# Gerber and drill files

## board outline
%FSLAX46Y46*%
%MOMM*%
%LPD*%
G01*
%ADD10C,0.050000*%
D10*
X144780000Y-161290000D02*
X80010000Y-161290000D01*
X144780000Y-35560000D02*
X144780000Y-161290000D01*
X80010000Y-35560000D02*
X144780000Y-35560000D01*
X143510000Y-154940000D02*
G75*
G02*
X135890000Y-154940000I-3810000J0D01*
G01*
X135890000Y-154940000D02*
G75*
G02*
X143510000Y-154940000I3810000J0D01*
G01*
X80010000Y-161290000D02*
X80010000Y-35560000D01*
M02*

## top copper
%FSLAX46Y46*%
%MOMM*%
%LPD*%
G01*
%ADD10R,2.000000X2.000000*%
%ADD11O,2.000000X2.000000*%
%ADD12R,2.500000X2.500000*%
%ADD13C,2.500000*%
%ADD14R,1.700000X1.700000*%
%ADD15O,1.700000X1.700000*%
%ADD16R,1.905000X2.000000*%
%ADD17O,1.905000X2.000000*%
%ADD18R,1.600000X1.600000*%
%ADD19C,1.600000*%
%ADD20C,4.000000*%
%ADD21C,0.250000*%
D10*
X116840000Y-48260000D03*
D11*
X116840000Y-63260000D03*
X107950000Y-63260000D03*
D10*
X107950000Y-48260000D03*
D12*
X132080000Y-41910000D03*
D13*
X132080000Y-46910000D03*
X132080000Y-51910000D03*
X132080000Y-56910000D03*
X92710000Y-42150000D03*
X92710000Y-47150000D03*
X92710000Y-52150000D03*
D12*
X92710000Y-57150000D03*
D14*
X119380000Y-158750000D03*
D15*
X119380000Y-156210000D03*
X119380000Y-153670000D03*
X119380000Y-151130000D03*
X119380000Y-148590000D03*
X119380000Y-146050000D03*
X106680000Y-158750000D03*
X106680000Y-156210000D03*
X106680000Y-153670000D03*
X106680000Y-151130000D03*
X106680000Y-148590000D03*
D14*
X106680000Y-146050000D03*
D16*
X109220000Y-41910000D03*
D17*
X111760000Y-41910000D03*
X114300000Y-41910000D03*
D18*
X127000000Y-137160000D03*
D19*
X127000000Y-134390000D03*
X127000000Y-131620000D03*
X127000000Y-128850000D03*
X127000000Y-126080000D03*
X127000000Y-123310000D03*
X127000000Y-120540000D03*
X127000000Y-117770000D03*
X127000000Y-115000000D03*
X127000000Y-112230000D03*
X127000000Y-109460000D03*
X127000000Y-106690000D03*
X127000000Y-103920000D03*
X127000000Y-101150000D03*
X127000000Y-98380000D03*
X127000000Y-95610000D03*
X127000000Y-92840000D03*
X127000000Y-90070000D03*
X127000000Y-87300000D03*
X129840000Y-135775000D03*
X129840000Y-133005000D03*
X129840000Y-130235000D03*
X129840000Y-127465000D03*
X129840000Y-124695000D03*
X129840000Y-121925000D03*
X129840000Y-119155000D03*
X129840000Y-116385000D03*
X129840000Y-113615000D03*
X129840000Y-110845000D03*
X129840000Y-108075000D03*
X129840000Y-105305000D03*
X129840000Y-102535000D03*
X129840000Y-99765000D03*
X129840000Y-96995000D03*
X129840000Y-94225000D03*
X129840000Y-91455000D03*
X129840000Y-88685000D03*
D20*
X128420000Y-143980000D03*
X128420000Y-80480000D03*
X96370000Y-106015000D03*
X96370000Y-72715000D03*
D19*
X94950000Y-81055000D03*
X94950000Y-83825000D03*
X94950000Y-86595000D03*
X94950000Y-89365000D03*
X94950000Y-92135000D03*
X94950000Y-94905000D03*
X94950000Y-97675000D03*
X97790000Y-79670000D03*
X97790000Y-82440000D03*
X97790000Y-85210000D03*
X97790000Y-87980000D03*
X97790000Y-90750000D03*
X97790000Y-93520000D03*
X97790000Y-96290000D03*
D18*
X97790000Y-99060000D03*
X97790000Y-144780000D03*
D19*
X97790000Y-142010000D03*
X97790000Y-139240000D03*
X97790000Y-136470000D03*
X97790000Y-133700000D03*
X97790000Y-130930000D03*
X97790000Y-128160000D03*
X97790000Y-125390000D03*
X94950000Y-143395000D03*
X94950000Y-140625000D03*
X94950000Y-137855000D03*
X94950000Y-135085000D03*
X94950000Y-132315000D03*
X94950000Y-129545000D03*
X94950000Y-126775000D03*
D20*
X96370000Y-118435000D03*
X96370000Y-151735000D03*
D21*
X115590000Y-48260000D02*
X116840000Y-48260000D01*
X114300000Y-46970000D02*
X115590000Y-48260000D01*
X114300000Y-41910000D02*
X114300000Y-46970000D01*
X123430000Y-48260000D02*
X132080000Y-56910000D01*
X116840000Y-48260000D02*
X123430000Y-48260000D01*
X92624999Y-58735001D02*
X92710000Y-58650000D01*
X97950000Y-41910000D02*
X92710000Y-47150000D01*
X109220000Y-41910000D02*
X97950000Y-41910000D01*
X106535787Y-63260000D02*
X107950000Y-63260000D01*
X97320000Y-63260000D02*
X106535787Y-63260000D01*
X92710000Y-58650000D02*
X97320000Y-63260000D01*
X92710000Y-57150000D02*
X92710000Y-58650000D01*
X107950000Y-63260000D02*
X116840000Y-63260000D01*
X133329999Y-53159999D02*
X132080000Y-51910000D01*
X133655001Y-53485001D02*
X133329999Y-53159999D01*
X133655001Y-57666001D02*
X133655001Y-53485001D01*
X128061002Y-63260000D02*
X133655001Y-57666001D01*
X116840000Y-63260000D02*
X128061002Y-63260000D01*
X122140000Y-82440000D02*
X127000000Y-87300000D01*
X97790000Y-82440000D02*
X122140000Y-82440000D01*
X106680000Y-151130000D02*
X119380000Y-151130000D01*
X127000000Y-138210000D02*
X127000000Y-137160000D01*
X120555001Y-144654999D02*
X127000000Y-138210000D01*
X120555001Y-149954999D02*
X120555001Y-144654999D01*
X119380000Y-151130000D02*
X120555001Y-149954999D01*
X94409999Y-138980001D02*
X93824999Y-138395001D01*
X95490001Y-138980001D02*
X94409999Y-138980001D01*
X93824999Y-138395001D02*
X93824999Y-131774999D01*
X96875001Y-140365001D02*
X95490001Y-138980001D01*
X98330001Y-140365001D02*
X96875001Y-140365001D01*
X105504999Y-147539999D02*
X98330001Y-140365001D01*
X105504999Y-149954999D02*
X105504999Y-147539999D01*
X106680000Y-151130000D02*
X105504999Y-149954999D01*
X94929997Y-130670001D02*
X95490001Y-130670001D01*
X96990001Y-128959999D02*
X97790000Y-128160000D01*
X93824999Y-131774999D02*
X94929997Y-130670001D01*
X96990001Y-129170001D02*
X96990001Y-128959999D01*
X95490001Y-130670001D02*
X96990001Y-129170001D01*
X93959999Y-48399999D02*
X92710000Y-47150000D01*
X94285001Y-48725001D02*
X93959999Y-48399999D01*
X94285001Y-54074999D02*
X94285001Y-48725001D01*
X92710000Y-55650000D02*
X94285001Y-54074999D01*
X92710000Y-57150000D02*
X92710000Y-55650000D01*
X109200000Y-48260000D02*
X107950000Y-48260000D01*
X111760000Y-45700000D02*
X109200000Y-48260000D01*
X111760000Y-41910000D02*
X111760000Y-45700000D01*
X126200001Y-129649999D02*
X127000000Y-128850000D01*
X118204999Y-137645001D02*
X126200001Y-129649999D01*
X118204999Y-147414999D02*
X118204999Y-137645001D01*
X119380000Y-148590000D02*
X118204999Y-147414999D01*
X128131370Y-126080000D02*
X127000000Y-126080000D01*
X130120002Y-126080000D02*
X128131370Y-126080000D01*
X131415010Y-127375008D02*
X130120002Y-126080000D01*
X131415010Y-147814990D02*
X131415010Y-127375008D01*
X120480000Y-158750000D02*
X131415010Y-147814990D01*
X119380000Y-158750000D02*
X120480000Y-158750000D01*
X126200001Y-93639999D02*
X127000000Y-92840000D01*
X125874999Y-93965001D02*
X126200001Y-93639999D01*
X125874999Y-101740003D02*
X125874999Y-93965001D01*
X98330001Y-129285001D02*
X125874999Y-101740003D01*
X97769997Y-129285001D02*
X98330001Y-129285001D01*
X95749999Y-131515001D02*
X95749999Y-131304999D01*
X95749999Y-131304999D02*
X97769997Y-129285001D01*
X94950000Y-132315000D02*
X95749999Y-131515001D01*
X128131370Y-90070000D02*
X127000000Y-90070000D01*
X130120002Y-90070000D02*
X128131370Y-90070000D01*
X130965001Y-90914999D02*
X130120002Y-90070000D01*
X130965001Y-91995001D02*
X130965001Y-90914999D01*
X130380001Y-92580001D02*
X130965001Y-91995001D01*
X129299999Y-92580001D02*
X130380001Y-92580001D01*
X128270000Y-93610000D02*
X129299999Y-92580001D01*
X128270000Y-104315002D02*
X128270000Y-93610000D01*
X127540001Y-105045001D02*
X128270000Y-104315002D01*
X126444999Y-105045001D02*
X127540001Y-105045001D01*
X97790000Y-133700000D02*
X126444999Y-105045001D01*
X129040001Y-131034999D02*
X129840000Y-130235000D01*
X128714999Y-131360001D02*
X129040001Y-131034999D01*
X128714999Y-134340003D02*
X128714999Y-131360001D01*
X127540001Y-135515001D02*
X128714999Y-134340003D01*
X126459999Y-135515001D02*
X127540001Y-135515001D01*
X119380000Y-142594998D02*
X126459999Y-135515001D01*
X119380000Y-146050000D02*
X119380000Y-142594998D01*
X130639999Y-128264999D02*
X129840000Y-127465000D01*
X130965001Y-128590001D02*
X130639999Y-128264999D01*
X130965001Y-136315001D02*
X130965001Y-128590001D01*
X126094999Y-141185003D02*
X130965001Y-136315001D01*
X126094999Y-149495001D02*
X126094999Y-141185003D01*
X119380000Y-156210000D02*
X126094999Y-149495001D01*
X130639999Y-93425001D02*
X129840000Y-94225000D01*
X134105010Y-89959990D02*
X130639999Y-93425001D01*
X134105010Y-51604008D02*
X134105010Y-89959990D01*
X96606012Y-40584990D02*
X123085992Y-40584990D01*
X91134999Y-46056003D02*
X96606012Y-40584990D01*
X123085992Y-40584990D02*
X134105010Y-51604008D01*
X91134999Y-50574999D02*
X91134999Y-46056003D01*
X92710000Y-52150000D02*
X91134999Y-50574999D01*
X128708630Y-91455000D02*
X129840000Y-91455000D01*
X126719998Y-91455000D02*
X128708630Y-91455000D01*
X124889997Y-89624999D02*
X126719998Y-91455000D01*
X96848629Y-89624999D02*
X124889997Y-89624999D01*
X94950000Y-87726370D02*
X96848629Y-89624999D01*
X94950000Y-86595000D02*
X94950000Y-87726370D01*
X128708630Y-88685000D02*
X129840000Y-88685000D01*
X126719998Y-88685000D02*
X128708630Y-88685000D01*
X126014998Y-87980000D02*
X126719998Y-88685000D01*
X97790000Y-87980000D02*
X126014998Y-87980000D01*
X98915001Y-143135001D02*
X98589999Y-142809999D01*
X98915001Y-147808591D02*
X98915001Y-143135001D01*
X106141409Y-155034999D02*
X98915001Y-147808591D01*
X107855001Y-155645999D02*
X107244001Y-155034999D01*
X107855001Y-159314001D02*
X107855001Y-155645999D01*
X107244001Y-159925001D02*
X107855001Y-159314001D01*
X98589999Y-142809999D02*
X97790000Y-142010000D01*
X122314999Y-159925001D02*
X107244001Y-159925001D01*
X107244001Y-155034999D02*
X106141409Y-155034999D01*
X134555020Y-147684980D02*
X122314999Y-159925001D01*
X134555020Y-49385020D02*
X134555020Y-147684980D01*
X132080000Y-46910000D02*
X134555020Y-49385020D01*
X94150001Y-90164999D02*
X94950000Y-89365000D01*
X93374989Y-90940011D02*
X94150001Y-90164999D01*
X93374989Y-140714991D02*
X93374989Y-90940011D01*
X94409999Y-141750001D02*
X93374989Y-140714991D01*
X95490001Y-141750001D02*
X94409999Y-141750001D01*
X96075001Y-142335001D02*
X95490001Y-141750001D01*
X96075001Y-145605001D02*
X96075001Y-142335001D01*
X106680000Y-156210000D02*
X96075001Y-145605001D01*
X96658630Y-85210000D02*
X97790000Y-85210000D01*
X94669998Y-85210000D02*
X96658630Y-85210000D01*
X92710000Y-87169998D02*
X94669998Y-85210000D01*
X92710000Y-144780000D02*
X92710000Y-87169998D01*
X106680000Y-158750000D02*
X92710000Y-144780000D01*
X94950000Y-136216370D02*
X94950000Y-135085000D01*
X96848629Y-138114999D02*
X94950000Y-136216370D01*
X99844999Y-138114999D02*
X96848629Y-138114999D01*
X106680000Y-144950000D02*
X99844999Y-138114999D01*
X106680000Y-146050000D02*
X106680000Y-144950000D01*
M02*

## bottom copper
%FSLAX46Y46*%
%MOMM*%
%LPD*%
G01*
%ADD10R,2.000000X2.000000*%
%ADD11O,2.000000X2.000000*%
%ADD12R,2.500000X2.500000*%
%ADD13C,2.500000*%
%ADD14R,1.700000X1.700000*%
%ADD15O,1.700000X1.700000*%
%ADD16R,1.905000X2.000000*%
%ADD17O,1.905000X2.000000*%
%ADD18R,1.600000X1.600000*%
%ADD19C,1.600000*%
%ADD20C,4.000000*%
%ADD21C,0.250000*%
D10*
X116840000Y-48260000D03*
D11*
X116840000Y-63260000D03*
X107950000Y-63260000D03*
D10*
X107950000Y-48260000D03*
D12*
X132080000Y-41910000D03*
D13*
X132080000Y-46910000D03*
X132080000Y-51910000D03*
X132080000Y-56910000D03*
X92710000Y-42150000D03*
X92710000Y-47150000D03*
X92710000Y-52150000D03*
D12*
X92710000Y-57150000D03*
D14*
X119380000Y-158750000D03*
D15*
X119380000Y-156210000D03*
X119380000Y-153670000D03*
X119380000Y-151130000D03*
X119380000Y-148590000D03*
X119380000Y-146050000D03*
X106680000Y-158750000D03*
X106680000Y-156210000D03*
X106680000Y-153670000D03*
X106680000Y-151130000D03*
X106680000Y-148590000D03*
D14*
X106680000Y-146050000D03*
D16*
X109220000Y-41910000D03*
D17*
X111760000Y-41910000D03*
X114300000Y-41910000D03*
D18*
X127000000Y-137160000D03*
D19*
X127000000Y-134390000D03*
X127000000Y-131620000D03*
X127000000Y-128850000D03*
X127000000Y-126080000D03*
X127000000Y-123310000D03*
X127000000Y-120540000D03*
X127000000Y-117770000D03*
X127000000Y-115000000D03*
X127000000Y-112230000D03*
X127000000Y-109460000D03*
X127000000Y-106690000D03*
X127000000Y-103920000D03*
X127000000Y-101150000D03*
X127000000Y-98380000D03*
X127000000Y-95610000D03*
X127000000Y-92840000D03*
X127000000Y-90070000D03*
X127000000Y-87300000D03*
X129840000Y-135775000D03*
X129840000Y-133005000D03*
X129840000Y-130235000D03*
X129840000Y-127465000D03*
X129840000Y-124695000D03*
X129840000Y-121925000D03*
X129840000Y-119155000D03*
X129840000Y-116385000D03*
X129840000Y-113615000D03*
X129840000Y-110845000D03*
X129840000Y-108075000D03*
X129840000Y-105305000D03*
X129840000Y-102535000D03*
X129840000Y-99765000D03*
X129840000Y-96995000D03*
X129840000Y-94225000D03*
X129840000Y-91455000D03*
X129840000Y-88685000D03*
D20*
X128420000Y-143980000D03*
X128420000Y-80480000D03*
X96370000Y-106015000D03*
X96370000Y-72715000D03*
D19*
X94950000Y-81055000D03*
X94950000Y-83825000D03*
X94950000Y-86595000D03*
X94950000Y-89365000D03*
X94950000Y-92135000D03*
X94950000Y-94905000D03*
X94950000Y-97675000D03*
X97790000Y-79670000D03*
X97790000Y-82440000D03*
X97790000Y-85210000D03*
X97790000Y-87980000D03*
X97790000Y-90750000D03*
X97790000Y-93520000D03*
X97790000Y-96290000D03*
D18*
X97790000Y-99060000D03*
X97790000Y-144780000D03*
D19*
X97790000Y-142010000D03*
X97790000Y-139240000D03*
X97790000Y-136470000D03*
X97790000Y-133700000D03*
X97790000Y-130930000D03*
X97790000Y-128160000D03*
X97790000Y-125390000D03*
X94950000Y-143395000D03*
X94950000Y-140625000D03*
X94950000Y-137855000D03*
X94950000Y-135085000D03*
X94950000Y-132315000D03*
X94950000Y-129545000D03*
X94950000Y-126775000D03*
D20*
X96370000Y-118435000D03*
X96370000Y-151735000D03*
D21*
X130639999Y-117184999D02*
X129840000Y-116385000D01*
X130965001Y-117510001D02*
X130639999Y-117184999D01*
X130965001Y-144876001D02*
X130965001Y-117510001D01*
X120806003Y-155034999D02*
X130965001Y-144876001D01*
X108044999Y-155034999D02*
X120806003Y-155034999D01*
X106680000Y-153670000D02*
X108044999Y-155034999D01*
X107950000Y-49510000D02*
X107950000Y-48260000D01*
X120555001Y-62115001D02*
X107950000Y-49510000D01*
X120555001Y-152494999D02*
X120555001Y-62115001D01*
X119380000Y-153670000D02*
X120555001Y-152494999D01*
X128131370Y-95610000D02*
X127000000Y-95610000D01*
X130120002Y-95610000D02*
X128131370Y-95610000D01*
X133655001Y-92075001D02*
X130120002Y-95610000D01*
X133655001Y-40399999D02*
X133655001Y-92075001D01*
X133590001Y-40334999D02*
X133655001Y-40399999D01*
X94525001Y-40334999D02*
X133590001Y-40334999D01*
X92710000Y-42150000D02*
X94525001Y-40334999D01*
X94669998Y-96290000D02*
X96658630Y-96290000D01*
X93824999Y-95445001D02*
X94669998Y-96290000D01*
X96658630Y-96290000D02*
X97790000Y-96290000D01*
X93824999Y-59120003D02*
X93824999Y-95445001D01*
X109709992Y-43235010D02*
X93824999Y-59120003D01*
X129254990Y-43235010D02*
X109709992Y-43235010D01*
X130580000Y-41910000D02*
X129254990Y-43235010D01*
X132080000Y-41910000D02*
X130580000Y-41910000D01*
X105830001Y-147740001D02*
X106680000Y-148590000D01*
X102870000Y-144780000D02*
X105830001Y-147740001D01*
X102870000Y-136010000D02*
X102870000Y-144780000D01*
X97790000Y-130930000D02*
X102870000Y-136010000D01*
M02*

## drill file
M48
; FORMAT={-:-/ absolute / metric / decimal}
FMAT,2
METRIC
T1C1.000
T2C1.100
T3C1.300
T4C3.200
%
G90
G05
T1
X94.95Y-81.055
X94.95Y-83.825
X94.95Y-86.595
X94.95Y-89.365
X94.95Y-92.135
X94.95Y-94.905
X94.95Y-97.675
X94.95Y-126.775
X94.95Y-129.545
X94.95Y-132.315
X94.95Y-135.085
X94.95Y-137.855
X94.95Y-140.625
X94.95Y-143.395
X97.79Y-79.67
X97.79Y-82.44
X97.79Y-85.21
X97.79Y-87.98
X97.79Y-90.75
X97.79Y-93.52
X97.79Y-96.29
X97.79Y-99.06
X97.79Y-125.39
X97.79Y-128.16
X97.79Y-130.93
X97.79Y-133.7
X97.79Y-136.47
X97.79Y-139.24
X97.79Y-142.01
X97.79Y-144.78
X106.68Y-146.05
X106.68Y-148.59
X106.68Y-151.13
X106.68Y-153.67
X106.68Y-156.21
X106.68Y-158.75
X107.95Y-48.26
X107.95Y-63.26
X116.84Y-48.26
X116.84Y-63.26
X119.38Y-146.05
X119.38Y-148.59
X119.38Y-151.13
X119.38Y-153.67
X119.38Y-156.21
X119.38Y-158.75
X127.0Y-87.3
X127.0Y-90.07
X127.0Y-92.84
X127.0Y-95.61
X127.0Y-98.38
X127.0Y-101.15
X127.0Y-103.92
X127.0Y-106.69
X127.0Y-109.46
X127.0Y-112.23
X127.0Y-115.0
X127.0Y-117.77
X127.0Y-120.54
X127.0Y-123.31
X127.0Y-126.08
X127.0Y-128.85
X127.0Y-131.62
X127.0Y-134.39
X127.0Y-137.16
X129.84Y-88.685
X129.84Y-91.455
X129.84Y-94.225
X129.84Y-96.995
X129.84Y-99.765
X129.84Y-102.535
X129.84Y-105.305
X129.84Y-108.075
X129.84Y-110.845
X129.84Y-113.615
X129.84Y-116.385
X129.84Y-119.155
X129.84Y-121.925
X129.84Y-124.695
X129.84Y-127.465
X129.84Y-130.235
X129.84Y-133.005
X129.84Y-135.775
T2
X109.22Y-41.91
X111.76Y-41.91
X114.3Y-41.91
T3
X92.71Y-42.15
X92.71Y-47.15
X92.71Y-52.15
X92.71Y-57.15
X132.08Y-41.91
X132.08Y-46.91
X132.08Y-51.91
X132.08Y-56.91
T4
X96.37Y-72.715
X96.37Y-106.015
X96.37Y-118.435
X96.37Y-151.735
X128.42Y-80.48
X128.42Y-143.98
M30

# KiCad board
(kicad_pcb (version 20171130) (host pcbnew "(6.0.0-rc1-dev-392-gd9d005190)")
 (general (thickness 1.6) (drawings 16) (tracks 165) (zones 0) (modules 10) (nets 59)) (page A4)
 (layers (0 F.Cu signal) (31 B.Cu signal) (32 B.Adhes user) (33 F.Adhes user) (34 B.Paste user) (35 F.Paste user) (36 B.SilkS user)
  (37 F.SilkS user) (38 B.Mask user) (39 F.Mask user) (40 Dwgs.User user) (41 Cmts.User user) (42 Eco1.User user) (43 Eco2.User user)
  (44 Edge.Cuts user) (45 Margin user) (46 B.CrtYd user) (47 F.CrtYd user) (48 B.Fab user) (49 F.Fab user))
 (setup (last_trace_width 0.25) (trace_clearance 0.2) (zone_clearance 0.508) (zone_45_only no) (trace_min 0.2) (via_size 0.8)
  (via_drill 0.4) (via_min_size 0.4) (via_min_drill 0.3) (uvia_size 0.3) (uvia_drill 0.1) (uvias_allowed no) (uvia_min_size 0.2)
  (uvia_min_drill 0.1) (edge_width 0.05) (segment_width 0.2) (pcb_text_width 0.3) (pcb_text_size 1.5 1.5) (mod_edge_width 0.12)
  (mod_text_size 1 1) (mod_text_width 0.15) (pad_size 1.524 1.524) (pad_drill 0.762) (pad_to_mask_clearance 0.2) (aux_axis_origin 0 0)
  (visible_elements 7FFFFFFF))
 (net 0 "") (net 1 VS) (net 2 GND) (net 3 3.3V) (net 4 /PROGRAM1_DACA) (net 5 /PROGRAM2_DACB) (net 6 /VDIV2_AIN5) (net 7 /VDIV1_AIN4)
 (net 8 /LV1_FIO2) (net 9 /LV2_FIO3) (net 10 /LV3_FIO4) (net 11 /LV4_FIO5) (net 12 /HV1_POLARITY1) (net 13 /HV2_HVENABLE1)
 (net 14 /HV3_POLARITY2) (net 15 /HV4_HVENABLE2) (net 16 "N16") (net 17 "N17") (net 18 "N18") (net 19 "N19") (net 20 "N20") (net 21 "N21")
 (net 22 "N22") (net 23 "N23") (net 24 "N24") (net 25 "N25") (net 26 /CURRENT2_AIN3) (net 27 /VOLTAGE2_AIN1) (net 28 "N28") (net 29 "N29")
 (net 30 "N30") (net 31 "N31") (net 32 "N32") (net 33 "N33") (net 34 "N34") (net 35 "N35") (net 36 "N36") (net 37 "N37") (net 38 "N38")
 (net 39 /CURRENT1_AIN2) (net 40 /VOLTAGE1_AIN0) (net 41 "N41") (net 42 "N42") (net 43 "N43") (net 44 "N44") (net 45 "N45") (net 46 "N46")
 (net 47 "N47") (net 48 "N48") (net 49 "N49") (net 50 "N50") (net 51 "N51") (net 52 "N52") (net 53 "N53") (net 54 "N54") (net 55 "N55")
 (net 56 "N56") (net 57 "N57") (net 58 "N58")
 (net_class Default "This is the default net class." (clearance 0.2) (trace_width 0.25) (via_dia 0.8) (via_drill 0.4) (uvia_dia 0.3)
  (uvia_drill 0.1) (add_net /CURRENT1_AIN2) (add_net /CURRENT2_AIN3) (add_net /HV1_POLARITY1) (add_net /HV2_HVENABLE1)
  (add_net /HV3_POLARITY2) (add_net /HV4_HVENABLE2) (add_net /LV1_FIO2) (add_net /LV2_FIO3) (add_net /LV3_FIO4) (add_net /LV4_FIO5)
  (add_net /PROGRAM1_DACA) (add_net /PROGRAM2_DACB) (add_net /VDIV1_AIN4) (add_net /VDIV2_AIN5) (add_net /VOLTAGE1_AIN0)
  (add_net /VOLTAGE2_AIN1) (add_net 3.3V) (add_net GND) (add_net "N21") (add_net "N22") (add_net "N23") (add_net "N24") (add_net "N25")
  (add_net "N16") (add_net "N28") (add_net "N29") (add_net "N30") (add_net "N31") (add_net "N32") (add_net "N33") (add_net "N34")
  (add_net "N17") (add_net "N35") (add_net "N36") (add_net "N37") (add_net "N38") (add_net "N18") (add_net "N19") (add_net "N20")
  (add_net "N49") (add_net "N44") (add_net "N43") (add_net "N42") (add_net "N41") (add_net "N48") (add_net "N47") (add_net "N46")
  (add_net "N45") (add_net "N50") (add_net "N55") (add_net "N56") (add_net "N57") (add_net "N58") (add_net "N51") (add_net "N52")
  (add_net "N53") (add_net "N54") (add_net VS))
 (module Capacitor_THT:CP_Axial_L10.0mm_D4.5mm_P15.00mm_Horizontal (layer F.Cu) (at 116.84 48.26 270)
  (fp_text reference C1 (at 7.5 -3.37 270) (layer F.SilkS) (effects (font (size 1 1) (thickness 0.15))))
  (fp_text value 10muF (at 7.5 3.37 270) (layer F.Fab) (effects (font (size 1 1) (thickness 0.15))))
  (pad 1 thru_hole rect (at 0 0 270) (size 2 2) (drill 1) (layers *.Cu *.Mask) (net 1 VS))
  (pad 2 thru_hole oval (at 15 0 270) (size 2 2) (drill 1) (layers *.Cu *.Mask) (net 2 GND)))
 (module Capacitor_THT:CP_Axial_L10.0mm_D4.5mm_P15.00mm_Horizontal (layer F.Cu) (at 107.95 48.26 270)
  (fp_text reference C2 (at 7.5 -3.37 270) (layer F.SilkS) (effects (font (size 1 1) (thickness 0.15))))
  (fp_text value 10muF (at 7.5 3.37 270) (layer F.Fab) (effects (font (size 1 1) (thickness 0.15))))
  (pad 2 thru_hole oval (at 15 0 270) (size 2 2) (drill 1) (layers *.Cu *.Mask) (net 2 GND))
  (pad 1 thru_hole rect (at 0 0 270) (size 2 2) (drill 1) (layers *.Cu *.Mask) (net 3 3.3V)))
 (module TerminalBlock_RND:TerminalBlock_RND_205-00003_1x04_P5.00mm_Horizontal (layer F.Cu) (at 132.08 41.91 270)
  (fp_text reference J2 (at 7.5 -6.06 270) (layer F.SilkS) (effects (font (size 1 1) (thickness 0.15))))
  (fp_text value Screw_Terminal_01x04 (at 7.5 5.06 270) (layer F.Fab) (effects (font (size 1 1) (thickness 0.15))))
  (pad 1 thru_hole rect (at 0 0 270) (size 2.5 2.5) (drill 1.3) (layers *.Cu *.Mask) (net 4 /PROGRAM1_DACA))
  (pad 2 thru_hole circle (at 5 0 270) (size 2.5 2.5) (drill 1.3) (layers *.Cu *.Mask) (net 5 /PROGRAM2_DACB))
  (pad 3 thru_hole circle (at 10 0 270) (size 2.5 2.5) (drill 1.3) (layers *.Cu *.Mask) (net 2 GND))
  (pad 4 thru_hole circle (at 15 0 270) (size 2.5 2.5) (drill 1.3) (layers *.Cu *.Mask) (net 1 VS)))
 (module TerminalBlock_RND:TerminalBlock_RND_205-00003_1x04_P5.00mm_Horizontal (layer F.Cu) (at 92.71 57.15 90)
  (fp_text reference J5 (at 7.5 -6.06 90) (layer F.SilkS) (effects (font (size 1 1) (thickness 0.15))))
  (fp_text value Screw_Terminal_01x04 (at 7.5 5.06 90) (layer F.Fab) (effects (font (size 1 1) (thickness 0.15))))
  (pad 4 thru_hole circle (at 15 0 90) (size 2.5 2.5) (drill 1.3) (layers *.Cu *.Mask) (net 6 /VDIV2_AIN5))
  (pad 3 thru_hole circle (at 10 0 90) (size 2.5 2.5) (drill 1.3) (layers *.Cu *.Mask) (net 2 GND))
  (pad 2 thru_hole circle (at 5 0 90) (size 2.5 2.5) (drill 1.3) (layers *.Cu *.Mask) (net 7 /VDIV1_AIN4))
  (pad 1 thru_hole rect (at 0 0 90) (size 2.5 2.5) (drill 1.3) (layers *.Cu *.Mask) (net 2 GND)))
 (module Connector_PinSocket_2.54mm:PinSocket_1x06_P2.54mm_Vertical (layer F.Cu) (at 119.38 158.75 180)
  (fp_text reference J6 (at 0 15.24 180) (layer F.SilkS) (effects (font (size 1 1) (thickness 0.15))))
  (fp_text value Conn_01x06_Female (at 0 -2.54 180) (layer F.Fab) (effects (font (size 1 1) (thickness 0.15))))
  (pad 1 thru_hole rect (at 0 0 180) (size 1.7 1.7) (drill 1) (layers *.Cu *.Mask) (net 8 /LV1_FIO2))
  (pad 2 thru_hole oval (at 0 2.54 180) (size 1.7 1.7) (drill 1) (layers *.Cu *.Mask) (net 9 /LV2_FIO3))
  (pad 3 thru_hole oval (at 0 5.08 180) (size 1.7 1.7) (drill 1) (layers *.Cu *.Mask) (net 3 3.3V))
  (pad 4 thru_hole oval (at 0 7.62 180) (size 1.7 1.7) (drill 1) (layers *.Cu *.Mask) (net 2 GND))
  (pad 5 thru_hole oval (at 0 10.16 180) (size 1.7 1.7) (drill 1) (layers *.Cu *.Mask) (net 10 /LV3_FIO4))
  (pad 6 thru_hole oval (at 0 12.7 180) (size 1.7 1.7) (drill 1) (layers *.Cu *.Mask) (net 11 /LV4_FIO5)))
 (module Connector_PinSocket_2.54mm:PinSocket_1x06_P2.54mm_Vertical (layer F.Cu) (at 106.68 146.05)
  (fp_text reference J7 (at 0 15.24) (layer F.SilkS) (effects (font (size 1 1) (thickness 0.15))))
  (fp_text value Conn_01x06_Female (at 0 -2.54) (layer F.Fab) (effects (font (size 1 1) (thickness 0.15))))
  (pad 6 thru_hole oval (at 0 12.7) (size 1.7 1.7) (drill 1) (layers *.Cu *.Mask) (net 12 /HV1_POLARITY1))
  (pad 5 thru_hole oval (at 0 10.16) (size 1.7 1.7) (drill 1) (layers *.Cu *.Mask) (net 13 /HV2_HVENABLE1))
  (pad 4 thru_hole oval (at 0 7.62) (size 1.7 1.7) (drill 1) (layers *.Cu *.Mask) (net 1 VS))
  (pad 3 thru_hole oval (at 0 5.08) (size 1.7 1.7) (drill 1) (layers *.Cu *.Mask) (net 2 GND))
  (pad 2 thru_hole oval (at 0 2.54) (size 1.7 1.7) (drill 1) (layers *.Cu *.Mask) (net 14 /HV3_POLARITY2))
  (pad 1 thru_hole rect (at 0 0) (size 1.7 1.7) (drill 1) (layers *.Cu *.Mask) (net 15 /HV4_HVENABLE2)))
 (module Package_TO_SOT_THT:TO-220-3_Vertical (layer F.Cu) (at 109.22 41.91)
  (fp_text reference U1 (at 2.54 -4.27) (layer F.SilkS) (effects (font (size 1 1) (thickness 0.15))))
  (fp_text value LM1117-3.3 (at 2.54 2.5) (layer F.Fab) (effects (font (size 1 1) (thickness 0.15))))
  (pad 1 thru_hole rect (at 0 0) (size 1.905 2) (drill 1.1) (layers *.Cu *.Mask) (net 2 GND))
  (pad 2 thru_hole oval (at 2.54 0) (size 1.905 2) (drill 1.1) (layers *.Cu *.Mask) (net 3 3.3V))
  (pad 3 thru_hole oval (at 5.08 0) (size 1.905 2) (drill 1.1) (layers *.Cu *.Mask) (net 1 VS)))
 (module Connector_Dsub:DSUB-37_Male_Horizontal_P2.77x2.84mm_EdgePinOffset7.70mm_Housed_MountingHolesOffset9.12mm (layer F.Cu)
  (at 127 137.16 90)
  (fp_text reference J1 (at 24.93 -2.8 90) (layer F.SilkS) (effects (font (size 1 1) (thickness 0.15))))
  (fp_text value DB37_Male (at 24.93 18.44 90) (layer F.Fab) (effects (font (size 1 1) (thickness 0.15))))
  (pad 1 thru_hole rect (at 0 0 90) (size 1.6 1.6) (drill 1) (layers *.Cu *.Mask) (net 2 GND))
  (pad 2 thru_hole circle (at 2.77 0 90) (size 1.6 1.6) (drill 1) (layers *.Cu *.Mask) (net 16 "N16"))
  (pad 3 thru_hole circle (at 5.54 0 90) (size 1.6 1.6) (drill 1) (layers *.Cu *.Mask) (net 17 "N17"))
  (pad 4 thru_hole circle (at 8.31 0 90) (size 1.6 1.6) (drill 1) (layers *.Cu *.Mask) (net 10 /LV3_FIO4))
  (pad 5 thru_hole circle (at 11.08 0 90) (size 1.6 1.6) (drill 1) (layers *.Cu *.Mask) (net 8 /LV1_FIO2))
  (pad 6 thru_hole circle (at 13.85 0 90) (size 1.6 1.6) (drill 1) (layers *.Cu *.Mask) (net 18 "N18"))
  (pad 7 thru_hole circle (at 16.62 0 90) (size 1.6 1.6) (drill 1) (layers *.Cu *.Mask) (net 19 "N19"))
  (pad 8 thru_hole circle (at 19.39 0 90) (size 1.6 1.6) (drill 1) (layers *.Cu *.Mask) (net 2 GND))
  (pad 9 thru_hole circle (at 22.16 0 90) (size 1.6 1.6) (drill 1) (layers *.Cu *.Mask) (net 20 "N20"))
  (pad 10 thru_hole circle (at 24.93 0 90) (size 1.6 1.6) (drill 1) (layers *.Cu *.Mask) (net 2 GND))
  (pad 11 thru_hole circle (at 27.7 0 90) (size 1.6 1.6) (drill 1) (layers *.Cu *.Mask) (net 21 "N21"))
  (pad 12 thru_hole circle (at 30.47 0 90) (size 1.6 1.6) (drill 1) (layers *.Cu *.Mask) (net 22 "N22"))
  (pad 13 thru_hole circle (at 33.24 0 90) (size 1.6 1.6) (drill 1) (layers *.Cu *.Mask) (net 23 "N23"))
  (pad 14 thru_hole circle (at 36.01 0 90) (size 1.6 1.6) (drill 1) (layers *.Cu *.Mask) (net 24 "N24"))
  (pad 15 thru_hole circle (at 38.78 0 90) (size 1.6 1.6) (drill 1) (layers *.Cu *.Mask) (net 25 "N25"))
  (pad 16 thru_hole circle (at 41.55 0 90) (size 1.6 1.6) (drill 1) (layers *.Cu *.Mask) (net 6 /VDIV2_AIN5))
  (pad 17 thru_hole circle (at 44.32 0 90) (size 1.6 1.6) (drill 1) (layers *.Cu *.Mask) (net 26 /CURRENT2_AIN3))
  (pad 18 thru_hole circle (at 47.09 0 90) (size 1.6 1.6) (drill 1) (layers *.Cu *.Mask) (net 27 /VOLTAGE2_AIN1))
  (pad 19 thru_hole circle (at 49.86 0 90) (size 1.6 1.6) (drill 1) (layers *.Cu *.Mask) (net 2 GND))
  (pad 20 thru_hole circle (at 1.385 2.84 90) (size 1.6 1.6) (drill 1) (layers *.Cu *.Mask) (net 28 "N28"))
  (pad 21 thru_hole circle (at 4.155 2.84 90) (size 1.6 1.6) (drill 1) (layers *.Cu *.Mask) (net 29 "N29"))
  (pad 22 thru_hole circle (at 6.925 2.84 90) (size 1.6 1.6) (drill 1) (layers *.Cu *.Mask) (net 11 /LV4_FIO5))
  (pad 23 thru_hole circle (at 9.695 2.84 90) (size 1.6 1.6) (drill 1) (layers *.Cu *.Mask) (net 9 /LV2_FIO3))
  (pad 24 thru_hole circle (at 12.465 2.84 90) (size 1.6 1.6) (drill 1) (layers *.Cu *.Mask) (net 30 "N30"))
  (pad 25 thru_hole circle (at 15.235 2.84 90) (size 1.6 1.6) (drill 1) (layers *.Cu *.Mask) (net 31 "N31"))
  (pad 26 thru_hole circle (at 18.005 2.84 90) (size 1.6 1.6) (drill 1) (layers *.Cu *.Mask) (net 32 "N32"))
  (pad 27 thru_hole circle (at 20.775 2.84 90) (size 1.6 1.6) (drill 1) (layers *.Cu *.Mask) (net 1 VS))
  (pad 28 thru_hole circle (at 23.545 2.84 90) (size 1.6 1.6) (drill 1) (layers *.Cu *.Mask) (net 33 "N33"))
  (pad 29 thru_hole circle (at 26.315 2.84 90) (size 1.6 1.6) (drill 1) (layers *.Cu *.Mask) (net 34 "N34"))
  (pad 30 thru_hole circle (at 29.085 2.84 90) (size 1.6 1.6) (drill 1) (layers *.Cu *.Mask) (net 2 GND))
  (pad 31 thru_hole circle (at 31.855 2.84 90) (size 1.6 1.6) (drill 1) (layers *.Cu *.Mask) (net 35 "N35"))
  (pad 32 thru_hole circle (at 34.625 2.84 90) (size 1.6 1.6) (drill 1) (layers *.Cu *.Mask) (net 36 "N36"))
  (pad 33 thru_hole circle (at 37.395 2.84 90) (size 1.6 1.6) (drill 1) (layers *.Cu *.Mask) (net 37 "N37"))
  (pad 34 thru_hole circle (at 40.165 2.84 90) (size 1.6 1.6) (drill 1) (layers *.Cu *.Mask) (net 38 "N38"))
  (pad 35 thru_hole circle (at 42.935 2.84 90) (size 1.6 1.6) (drill 1) (layers *.Cu *.Mask) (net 7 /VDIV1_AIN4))
  (pad 36 thru_hole circle (at 45.705 2.84 90) (size 1.6 1.6) (drill 1) (layers *.Cu *.Mask) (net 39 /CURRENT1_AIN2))
  (pad 37 thru_hole circle (at 48.475 2.84 90) (size 1.6 1.6) (drill 1) (layers *.Cu *.Mask) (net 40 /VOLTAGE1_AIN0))
  (pad 0 thru_hole circle (at -6.82 1.42 90) (size 4 4) (drill 3.2) (layers *.Cu *.Mask))
  (pad 0 thru_hole circle (at 56.68 1.42 90) (size 4 4) (drill 3.2) (layers *.Cu *.Mask)))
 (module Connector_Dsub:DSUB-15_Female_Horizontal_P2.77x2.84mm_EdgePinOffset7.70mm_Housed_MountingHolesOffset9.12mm (layer F.Cu)
  (at 97.79 99.06 270)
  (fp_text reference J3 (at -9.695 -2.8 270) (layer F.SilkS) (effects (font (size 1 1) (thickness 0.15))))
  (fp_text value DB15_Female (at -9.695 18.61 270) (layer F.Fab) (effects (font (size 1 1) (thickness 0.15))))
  (pad 0 thru_hole circle (at 6.955 1.42 270) (size 4 4) (drill 3.2) (layers *.Cu *.Mask))
  (pad 0 thru_hole circle (at -26.345 1.42 270) (size 4 4) (drill 3.2) (layers *.Cu *.Mask))
  (pad 15 thru_hole circle (at -18.005 2.84 270) (size 1.6 1.6) (drill 1) (layers *.Cu *.Mask) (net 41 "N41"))
  (pad 14 thru_hole circle (at -15.235 2.84 270) (size 1.6 1.6) (drill 1) (layers *.Cu *.Mask) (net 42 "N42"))
  (pad 13 thru_hole circle (at -12.465 2.84 270) (size 1.6 1.6) (drill 1) (layers *.Cu *.Mask) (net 39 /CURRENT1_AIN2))
  (pad 12 thru_hole circle (at -9.695 2.84 270) (size 1.6 1.6) (drill 1) (layers *.Cu *.Mask) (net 13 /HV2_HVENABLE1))
  (pad 11 thru_hole circle (at -6.925 2.84 270) (size 1.6 1.6) (drill 1) (layers *.Cu *.Mask) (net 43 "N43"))
  (pad 10 thru_hole circle (at -4.155 2.84 270) (size 1.6 1.6) (drill 1) (layers *.Cu *.Mask) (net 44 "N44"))
  (pad 9 thru_hole circle (at -1.385 2.84 270) (size 1.6 1.6) (drill 1) (layers *.Cu *.Mask) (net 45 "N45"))
  (pad 8 thru_hole circle (at -19.39 0 270) (size 1.6 1.6) (drill 1) (layers *.Cu *.Mask) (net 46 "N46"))
  (pad 7 thru_hole circle (at -16.62 0 270) (size 1.6 1.6) (drill 1) (layers *.Cu *.Mask) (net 2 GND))
  (pad 6 thru_hole circle (at -13.85 0 270) (size 1.6 1.6) (drill 1) (layers *.Cu *.Mask) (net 12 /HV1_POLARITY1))
  (pad 5 thru_hole circle (at -11.08 0 270) (size 1.6 1.6) (drill 1) (layers *.Cu *.Mask) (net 40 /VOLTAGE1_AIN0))
  (pad 4 thru_hole circle (at -8.31 0 270) (size 1.6 1.6) (drill 1) (layers *.Cu *.Mask) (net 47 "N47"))
  (pad 3 thru_hole circle (at -5.54 0 270) (size 1.6 1.6) (drill 1) (layers *.Cu *.Mask) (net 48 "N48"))
  (pad 2 thru_hole circle (at -2.77 0 270) (size 1.6 1.6) (drill 1) (layers *.Cu *.Mask) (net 4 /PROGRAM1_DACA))
  (pad 1 thru_hole rect (at 0 0 270) (size 1.6 1.6) (drill 1) (layers *.Cu *.Mask) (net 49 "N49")))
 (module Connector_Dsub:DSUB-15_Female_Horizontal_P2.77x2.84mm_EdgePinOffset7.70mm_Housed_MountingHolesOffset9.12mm (layer F.Cu)
  (at 97.79 144.78 270)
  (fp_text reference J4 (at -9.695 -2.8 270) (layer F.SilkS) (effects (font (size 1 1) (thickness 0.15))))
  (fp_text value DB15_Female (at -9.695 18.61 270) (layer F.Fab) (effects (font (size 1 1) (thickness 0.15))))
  (pad 1 thru_hole rect (at 0 0 270) (size 1.6 1.6) (drill 1) (layers *.Cu *.Mask) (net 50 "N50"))
  (pad 2 thru_hole circle (at -2.77 0 270) (size 1.6 1.6) (drill 1) (layers *.Cu *.Mask) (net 5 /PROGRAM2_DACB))
  (pad 3 thru_hole circle (at -5.54 0 270) (size 1.6 1.6) (drill 1) (layers *.Cu *.Mask) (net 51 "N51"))
  (pad 4 thru_hole circle (at -8.31 0 270) (size 1.6 1.6) (drill 1) (layers *.Cu *.Mask) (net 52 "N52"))
  (pad 5 thru_hole circle (at -11.08 0 270) (size 1.6 1.6) (drill 1) (layers *.Cu *.Mask) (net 27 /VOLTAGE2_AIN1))
  (pad 6 thru_hole circle (at -13.85 0 270) (size 1.6 1.6) (drill 1) (layers *.Cu *.Mask) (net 14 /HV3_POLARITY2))
  (pad 7 thru_hole circle (at -16.62 0 270) (size 1.6 1.6) (drill 1) (layers *.Cu *.Mask) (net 2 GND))
  (pad 8 thru_hole circle (at -19.39 0 270) (size 1.6 1.6) (drill 1) (layers *.Cu *.Mask) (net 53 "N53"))
  (pad 9 thru_hole circle (at -1.385 2.84 270) (size 1.6 1.6) (drill 1) (layers *.Cu *.Mask) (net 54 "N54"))
  (pad 10 thru_hole circle (at -4.155 2.84 270) (size 1.6 1.6) (drill 1) (layers *.Cu *.Mask) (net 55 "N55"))
  (pad 11 thru_hole circle (at -6.925 2.84 270) (size 1.6 1.6) (drill 1) (layers *.Cu *.Mask) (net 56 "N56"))
  (pad 12 thru_hole circle (at -9.695 2.84 270) (size 1.6 1.6) (drill 1) (layers *.Cu *.Mask) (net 15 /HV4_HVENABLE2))
  (pad 13 thru_hole circle (at -12.465 2.84 270) (size 1.6 1.6) (drill 1) (layers *.Cu *.Mask) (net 26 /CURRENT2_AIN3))
  (pad 14 thru_hole circle (at -15.235 2.84 270) (size 1.6 1.6) (drill 1) (layers *.Cu *.Mask) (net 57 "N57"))
  (pad 15 thru_hole circle (at -18.005 2.84 270) (size 1.6 1.6) (drill 1) (layers *.Cu *.Mask) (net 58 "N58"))
  (pad 0 thru_hole circle (at -26.345 1.42 270) (size 4 4) (drill 3.2) (layers *.Cu *.Mask))
  (pad 0 thru_hole circle (at 6.955 1.42 270) (size 4 4) (drill 3.2) (layers *.Cu *.Mask)))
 (gr_line (start 144.78 161.29) (end 80.01 161.29) (layer Edge.Cuts) (width 0.05))
 (gr_line (start 144.78 35.56) (end 144.78 161.29) (layer Edge.Cuts) (width 0.05))
 (gr_line (start 80.01 35.56) (end 144.78 35.56) (layer Edge.Cuts) (width 0.05))
 (gr_circle (center 139.7 154.94) (end 143.51 154.94) (layer Edge.Cuts) (width 0.05))
 (gr_line (start 80.01 161.29) (end 80.01 35.56) (layer Edge.Cuts) (width 0.05))
 (segment (start 115.59 48.26) (end 116.84 48.26) (width 0.25) (layer F.Cu) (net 1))
 (segment (start 114.3 46.97) (end 115.59 48.26) (width 0.25) (layer F.Cu) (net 1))
 (segment (start 114.3 41.91) (end 114.3 46.97) (width 0.25) (layer F.Cu) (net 1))
 (segment (start 123.43 48.26) (end 132.08 56.91) (width 0.25) (layer F.Cu) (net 1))
 (segment (start 116.84 48.26) (end 123.43 48.26) (width 0.25) (layer F.Cu) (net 1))
 (segment (start 130.639999 117.184999) (end 129.84 116.385) (width 0.25) (layer B.Cu) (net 1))
 (segment (start 130.965001 117.510001) (end 130.639999 117.184999) (width 0.25) (layer B.Cu) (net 1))
 (segment (start 130.965001 144.876001) (end 130.965001 117.510001) (width 0.25) (layer B.Cu) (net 1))
 (segment (start 120.806003 155.034999) (end 130.965001 144.876001) (width 0.25) (layer B.Cu) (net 1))
 (segment (start 108.044999 155.034999) (end 120.806003 155.034999) (width 0.25) (layer B.Cu) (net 1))
 (segment (start 106.68 153.67) (end 108.044999 155.034999) (width 0.25) (layer B.Cu) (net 1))
 (segment (start 92.624999 58.735001) (end 92.71 58.65) (width 0.25) (layer F.Cu) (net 2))
 (segment (start 97.95 41.91) (end 92.71 47.15) (width 0.25) (layer F.Cu) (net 2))
 (segment (start 109.22 41.91) (end 97.95 41.91) (width 0.25) (layer F.Cu) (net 2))
 (segment (start 106.535787 63.26) (end 107.95 63.26) (width 0.25) (layer F.Cu) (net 2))
 (segment (start 97.32 63.26) (end 106.535787 63.26) (width 0.25) (layer F.Cu) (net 2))
 (segment (start 92.71 58.65) (end 97.32 63.26) (width 0.25) (layer F.Cu) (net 2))
 (segment (start 92.71 57.15) (end 92.71 58.65) (width 0.25) (layer F.Cu) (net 2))
 (segment (start 107.95 63.26) (end 116.84 63.26) (width 0.25) (layer F.Cu) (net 2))
 (segment (start 133.329999 53.159999) (end 132.08 51.91) (width 0.25) (layer F.Cu) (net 2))
 (segment (start 133.655001 53.485001) (end 133.329999 53.159999) (width 0.25) (layer F.Cu) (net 2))
 (segment (start 133.655001 57.666001) (end 133.655001 53.485001) (width 0.25) (layer F.Cu) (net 2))
 (segment (start 128.061002 63.26) (end 133.655001 57.666001) (width 0.25) (layer F.Cu) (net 2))
 (segment (start 116.84 63.26) (end 128.061002 63.26) (width 0.25) (layer F.Cu) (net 2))
 (segment (start 122.14 82.44) (end 127 87.3) (width 0.25) (layer F.Cu) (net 2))
 (segment (start 97.79 82.44) (end 122.14 82.44) (width 0.25) (layer F.Cu) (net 2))
 (segment (start 106.68 151.13) (end 119.38 151.13) (width 0.25) (layer F.Cu) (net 2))
 (segment (start 127 138.21) (end 127 137.16) (width 0.25) (layer F.Cu) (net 2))
 (segment (start 120.555001 144.654999) (end 127 138.21) (width 0.25) (layer F.Cu) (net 2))
 (segment (start 120.555001 149.954999) (end 120.555001 144.654999) (width 0.25) (layer F.Cu) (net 2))
 (segment (start 119.38 151.13) (end 120.555001 149.954999) (width 0.25) (layer F.Cu) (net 2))
 (segment (start 94.409999 138.980001) (end 93.824999 138.395001) (width 0.25) (layer F.Cu) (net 2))
 (segment (start 95.490001 138.980001) (end 94.409999 138.980001) (width 0.25) (layer F.Cu) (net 2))
 (segment (start 93.824999 138.395001) (end 93.824999 131.774999) (width 0.25) (layer F.Cu) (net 2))
 (segment (start 96.875001 140.365001) (end 95.490001 138.980001) (width 0.25) (layer F.Cu) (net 2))
 (segment (start 98.330001 140.365001) (end 96.875001 140.365001) (width 0.25) (layer F.Cu) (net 2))
 (segment (start 105.504999 147.539999) (end 98.330001 140.365001) (width 0.25) (layer F.Cu) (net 2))
 (segment (start 105.504999 149.954999) (end 105.504999 147.539999) (width 0.25) (layer F.Cu) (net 2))
 (segment (start 106.68 151.13) (end 105.504999 149.954999) (width 0.25) (layer F.Cu) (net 2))
 (segment (start 94.929997 130.670001) (end 95.490001 130.670001) (width 0.25) (layer F.Cu) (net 2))
 (segment (start 96.990001 128.959999) (end 97.79 128.16) (width 0.25) (layer F.Cu) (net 2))
 (segment (start 93.824999 131.774999) (end 94.929997 130.670001) (width 0.25) (layer F.Cu) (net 2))
 (segment (start 96.990001 129.170001) (end 96.990001 128.959999) (width 0.25) (layer F.Cu) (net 2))
 (segment (start 95.490001 130.670001) (end 96.990001 129.170001) (width 0.25) (layer F.Cu) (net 2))
 (segment (start 93.959999 48.399999) (end 92.71 47.15) (width 0.25) (layer F.Cu) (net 2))
 (segment (start 94.285001 48.725001) (end 93.959999 48.399999) (width 0.25) (layer F.Cu) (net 2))
 (segment (start 94.285001 54.074999) (end 94.285001 48.725001) (width 0.25) (layer F.Cu) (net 2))
 (segment (start 92.71 55.65) (end 94.285001 54.074999) (width 0.25) (layer F.Cu) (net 2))
 (segment (start 92.71 57.15) (end 92.71 55.65) (width 0.25) (layer F.Cu) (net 2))
 (segment (start 109.2 48.26) (end 107.95 48.26) (width 0.25) (layer F.Cu) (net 3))
 (segment (start 111.76 45.7) (end 109.2 48.26) (width 0.25) (layer F.Cu) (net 3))
 (segment (start 111.76 41.91) (end 111.76 45.7) (width 0.25) (layer F.Cu) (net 3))
 (segment (start 107.95 49.51) (end 107.95 48.26) (width 0.25) (layer B.Cu) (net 3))
 (segment (start 120.555001 62.115001) (end 107.95 49.51) (width 0.25) (layer B.Cu) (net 3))
 (segment (start 120.555001 152.494999) (end 120.555001 62.115001) (width 0.25) (layer B.Cu) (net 3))
 (segment (start 119.38 153.67) (end 120.555001 152.494999) (width 0.25) (layer B.Cu) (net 3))
 (segment (start 126.200001 129.649999) (end 127 128.85) (width 0.25) (layer F.Cu) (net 10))
 (segment (start 118.204999 137.645001) (end 126.200001 129.649999) (width 0.25) (layer F.Cu) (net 10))
 (segment (start 118.204999 147.414999) (end 118.204999 137.645001) (width 0.25) (layer F.Cu) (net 10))
 (segment (start 119.38 148.59) (end 118.204999 147.414999) (width 0.25) (layer F.Cu) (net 10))
 (segment (start 128.13137 126.08) (end 127 126.08) (width 0.25) (layer F.Cu) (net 8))
 (segment (start 130.120002 126.08) (end 128.13137 126.08) (width 0.25) (layer F.Cu) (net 8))
 (segment (start 131.41501 127.375008) (end 130.120002 126.08) (width 0.25) (layer F.Cu) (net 8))
 (segment (start 131.41501 147.81499) (end 131.41501 127.375008) (width 0.25) (layer F.Cu) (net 8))
 (segment (start 120.48 158.75) (end 131.41501 147.81499) (width 0.25) (layer F.Cu) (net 8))
 (segment (start 119.38 158.75) (end 120.48 158.75) (width 0.25) (layer F.Cu) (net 8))
 (segment (start 128.13137 95.61) (end 127 95.61) (width 0.25) (layer B.Cu) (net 6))
 (segment (start 130.120002 95.61) (end 128.13137 95.61) (width 0.25) (layer B.Cu) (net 6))
 (segment (start 133.655001 92.075001) (end 130.120002 95.61) (width 0.25) (layer B.Cu) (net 6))
 (segment (start 133.655001 40.399999) (end 133.655001 92.075001) (width 0.25) (layer B.Cu) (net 6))
 (segment (start 133.590001 40.334999) (end 133.655001 40.399999) (width 0.25) (layer B.Cu) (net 6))
 (segment (start 94.525001 40.334999) (end 133.590001 40.334999) (width 0.25) (layer B.Cu) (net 6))
 (segment (start 92.71 42.15) (end 94.525001 40.334999) (width 0.25) (layer B.Cu) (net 6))
 (segment (start 126.200001 93.639999) (end 127 92.84) (width 0.25) (layer F.Cu) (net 26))
 (segment (start 125.874999 93.965001) (end 126.200001 93.639999) (width 0.25) (layer F.Cu) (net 26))
 (segment (start 125.874999 101.740003) (end 125.874999 93.965001) (width 0.25) (layer F.Cu) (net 26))
 (segment (start 98.330001 129.285001) (end 125.874999 101.740003) (width 0.25) (layer F.Cu) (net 26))
 (segment (start 97.769997 129.285001) (end 98.330001 129.285001) (width 0.25) (layer F.Cu) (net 26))
 (segment (start 95.749999 131.515001) (end 95.749999 131.304999) (width 0.25) (layer F.Cu) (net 26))
 (segment (start 95.749999 131.304999) (end 97.769997 129.285001) (width 0.25) (layer F.Cu) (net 26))
 (segment (start 94.95 132.315) (end 95.749999 131.515001) (width 0.25) (layer F.Cu) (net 26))
 (segment (start 128.13137 90.07) (end 127 90.07) (width 0.25) (layer F.Cu) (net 27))
 (segment (start 130.120002 90.07) (end 128.13137 90.07) (width 0.25) (layer F.Cu) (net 27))
 (segment (start 130.965001 90.914999) (end 130.120002 90.07) (width 0.25) (layer F.Cu) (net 27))
 (segment (start 130.965001 91.995001) (end 130.965001 90.914999) (width 0.25) (layer F.Cu) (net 27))
 (segment (start 130.380001 92.580001) (end 130.965001 91.995001) (width 0.25) (layer F.Cu) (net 27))
 (segment (start 129.299999 92.580001) (end 130.380001 92.580001) (width 0.25) (layer F.Cu) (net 27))
 (segment (start 128.27 93.61) (end 129.299999 92.580001) (width 0.25) (layer F.Cu) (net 27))
 (segment (start 128.27 104.315002) (end 128.27 93.61) (width 0.25) (layer F.Cu) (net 27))
 (segment (start 127.540001 105.045001) (end 128.27 104.315002) (width 0.25) (layer F.Cu) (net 27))
 (segment (start 126.444999 105.045001) (end 127.540001 105.045001) (width 0.25) (layer F.Cu) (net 27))
 (segment (start 97.79 133.7) (end 126.444999 105.045001) (width 0.25) (layer F.Cu) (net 27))
 (segment (start 129.040001 131.034999) (end 129.84 130.235) (width 0.25) (layer F.Cu) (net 11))
 (segment (start 128.714999 131.360001) (end 129.040001 131.034999) (width 0.25) (layer F.Cu) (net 11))
 (segment (start 128.714999 134.340003) (end 128.714999 131.360001) (width 0.25) (layer F.Cu) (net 11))
 (segment (start 127.540001 135.515001) (end 128.714999 134.340003) (width 0.25) (layer F.Cu) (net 11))
 (segment (start 126.459999 135.515001) (end 127.540001 135.515001) (width 0.25) (layer F.Cu) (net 11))
 (segment (start 119.38 142.594998) (end 126.459999 135.515001) (width 0.25) (layer F.Cu) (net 11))
 (segment (start 119.38 146.05) (end 119.38 142.594998) (width 0.25) (layer F.Cu) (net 11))
 (segment (start 130.639999 128.264999) (end 129.84 127.465) (width 0.25) (layer F.Cu) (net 9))
 (segment (start 130.965001 128.590001) (end 130.639999 128.264999) (width 0.25) (layer F.Cu) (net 9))
 (segment (start 130.965001 136.315001) (end 130.965001 128.590001) (width 0.25) (layer F.Cu) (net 9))
 (segment (start 126.094999 141.185003) (end 130.965001 136.315001) (width 0.25) (layer F.Cu) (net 9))
 (segment (start 126.094999 149.495001) (end 126.094999 141.185003) (width 0.25) (layer F.Cu) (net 9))
 (segment (start 119.38 156.21) (end 126.094999 149.495001) (width 0.25) (layer F.Cu) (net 9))
 (segment (start 130.639999 93.425001) (end 129.84 94.225) (width 0.25) (layer F.Cu) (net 7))
 (segment (start 134.10501 89.95999) (end 130.639999 93.425001) (width 0.25) (layer F.Cu) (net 7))
 (segment (start 134.10501 51.604008) (end 134.10501 89.95999) (width 0.25) (layer F.Cu) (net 7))
 (segment (start 96.606012 40.58499) (end 123.085992 40.58499) (width 0.25) (layer F.Cu) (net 7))
 (segment (start 91.134999 46.056003) (end 96.606012 40.58499) (width 0.25) (layer F.Cu) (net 7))
 (segment (start 123.085992 40.58499) (end 134.10501 51.604008) (width 0.25) (layer F.Cu) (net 7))
 (segment (start 91.134999 50.574999) (end 91.134999 46.056003) (width 0.25) (layer F.Cu) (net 7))
 (segment (start 92.71 52.15) (end 91.134999 50.574999) (width 0.25) (layer F.Cu) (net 7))
 (segment (start 128.70863 91.455) (end 129.84 91.455) (width 0.25) (layer F.Cu) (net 39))
 (segment (start 126.719998 91.455) (end 128.70863 91.455) (width 0.25) (layer F.Cu) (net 39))
 (segment (start 124.889997 89.624999) (end 126.719998 91.455) (width 0.25) (layer F.Cu) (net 39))
 (segment (start 96.848629 89.624999) (end 124.889997 89.624999) (width 0.25) (layer F.Cu) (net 39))
 (segment (start 94.95 87.72637) (end 96.848629 89.624999) (width 0.25) (layer F.Cu) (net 39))
 (segment (start 94.95 86.595) (end 94.95 87.72637) (width 0.25) (layer F.Cu) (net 39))
 (segment (start 128.70863 88.685) (end 129.84 88.685) (width 0.25) (layer F.Cu) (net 40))
 (segment (start 126.719998 88.685) (end 128.70863 88.685) (width 0.25) (layer F.Cu) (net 40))
 (segment (start 126.014998 87.98) (end 126.719998 88.685) (width 0.25) (layer F.Cu) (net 40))
 (segment (start 97.79 87.98) (end 126.014998 87.98) (width 0.25) (layer F.Cu) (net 40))
 (segment (start 94.669998 96.29) (end 96.65863 96.29) (width 0.25) (layer B.Cu) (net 4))
 (segment (start 93.824999 95.445001) (end 94.669998 96.29) (width 0.25) (layer B.Cu) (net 4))
 (segment (start 96.65863 96.29) (end 97.79 96.29) (width 0.25) (layer B.Cu) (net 4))
 (segment (start 93.824999 59.120003) (end 93.824999 95.445001) (width 0.25) (layer B.Cu) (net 4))
 (segment (start 109.709992 43.23501) (end 93.824999 59.120003) (width 0.25) (layer B.Cu) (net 4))
 (segment (start 129.25499 43.23501) (end 109.709992 43.23501) (width 0.25) (layer B.Cu) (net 4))
 (segment (start 130.58 41.91) (end 129.25499 43.23501) (width 0.25) (layer B.Cu) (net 4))
 (segment (start 132.08 41.91) (end 130.58 41.91) (width 0.25) (layer B.Cu) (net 4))
 (segment (start 98.915001 143.135001) (end 98.589999 142.809999) (width 0.25) (layer F.Cu) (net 5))
 (segment (start 98.915001 147.808591) (end 98.915001 143.135001) (width 0.25) (layer F.Cu) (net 5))
 (segment (start 106.141409 155.034999) (end 98.915001 147.808591) (width 0.25) (layer F.Cu) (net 5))
 (segment (start 107.855001 155.645999) (end 107.244001 155.034999) (width 0.25) (layer F.Cu) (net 5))
 (segment (start 107.855001 159.314001) (end 107.855001 155.645999) (width 0.25) (layer F.Cu) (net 5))
 (segment (start 107.244001 159.925001) (end 107.855001 159.314001) (width 0.25) (layer F.Cu) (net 5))
 (segment (start 98.589999 142.809999) (end 97.79 142.01) (width 0.25) (layer F.Cu) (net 5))
 (segment (start 122.314999 159.925001) (end 107.244001 159.925001) (width 0.25) (layer F.Cu) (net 5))
 (segment (start 107.244001 155.034999) (end 106.141409 155.034999) (width 0.25) (layer F.Cu) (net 5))
 (segment (start 134.55502 147.68498) (end 122.314999 159.925001) (width 0.25) (layer F.Cu) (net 5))
 (segment (start 134.55502 49.38502) (end 134.55502 147.68498) (width 0.25) (layer F.Cu) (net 5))
 (segment (start 132.08 46.91) (end 134.55502 49.38502) (width 0.25) (layer F.Cu) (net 5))
 (segment (start 94.150001 90.164999) (end 94.95 89.365) (width 0.25) (layer F.Cu) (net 13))
 (segment (start 93.374989 90.940011) (end 94.150001 90.164999) (width 0.25) (layer F.Cu) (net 13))
 (segment (start 93.374989 140.714991) (end 93.374989 90.940011) (width 0.25) (layer F.Cu) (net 13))
 (segment (start 94.409999 141.750001) (end 93.374989 140.714991) (width 0.25) (layer F.Cu) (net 13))
 (segment (start 95.490001 141.750001) (end 94.409999 141.750001) (width 0.25) (layer F.Cu) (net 13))
 (segment (start 96.075001 142.335001) (end 95.490001 141.750001) (width 0.25) (layer F.Cu) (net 13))
 (segment (start 96.075001 145.605001) (end 96.075001 142.335001) (width 0.25) (layer F.Cu) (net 13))
 (segment (start 106.68 156.21) (end 96.075001 145.605001) (width 0.25) (layer F.Cu) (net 13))
 (segment (start 96.65863 85.21) (end 97.79 85.21) (width 0.25) (layer F.Cu) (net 12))
 (segment (start 94.669998 85.21) (end 96.65863 85.21) (width 0.25) (layer F.Cu) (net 12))
 (segment (start 92.71 87.169998) (end 94.669998 85.21) (width 0.25) (layer F.Cu) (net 12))
 (segment (start 92.71 144.78) (end 92.71 87.169998) (width 0.25) (layer F.Cu) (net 12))
 (segment (start 106.68 158.75) (end 92.71 144.78) (width 0.25) (layer F.Cu) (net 12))
 (segment (start 105.830001 147.740001) (end 106.68 148.59) (width 0.25) (layer B.Cu) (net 14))
 (segment (start 102.87 144.78) (end 105.830001 147.740001) (width 0.25) (layer B.Cu) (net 14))
 (segment (start 102.87 136.01) (end 102.87 144.78) (width 0.25) (layer B.Cu) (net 14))
 (segment (start 97.79 130.93) (end 102.87 136.01) (width 0.25) (layer B.Cu) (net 14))
 (segment (start 94.95 136.21637) (end 94.95 135.085) (width 0.25) (layer F.Cu) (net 15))
 (segment (start 96.848629 138.114999) (end 94.95 136.21637) (width 0.25) (layer F.Cu) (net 15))
 (segment (start 99.844999 138.114999) (end 96.848629 138.114999) (width 0.25) (layer F.Cu) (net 15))
 (segment (start 106.68 144.95) (end 99.844999 138.114999) (width 0.25) (layer F.Cu) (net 15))
 (segment (start 106.68 146.05) (end 106.68 144.95) (width 0.25) (layer F.Cu) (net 15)))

